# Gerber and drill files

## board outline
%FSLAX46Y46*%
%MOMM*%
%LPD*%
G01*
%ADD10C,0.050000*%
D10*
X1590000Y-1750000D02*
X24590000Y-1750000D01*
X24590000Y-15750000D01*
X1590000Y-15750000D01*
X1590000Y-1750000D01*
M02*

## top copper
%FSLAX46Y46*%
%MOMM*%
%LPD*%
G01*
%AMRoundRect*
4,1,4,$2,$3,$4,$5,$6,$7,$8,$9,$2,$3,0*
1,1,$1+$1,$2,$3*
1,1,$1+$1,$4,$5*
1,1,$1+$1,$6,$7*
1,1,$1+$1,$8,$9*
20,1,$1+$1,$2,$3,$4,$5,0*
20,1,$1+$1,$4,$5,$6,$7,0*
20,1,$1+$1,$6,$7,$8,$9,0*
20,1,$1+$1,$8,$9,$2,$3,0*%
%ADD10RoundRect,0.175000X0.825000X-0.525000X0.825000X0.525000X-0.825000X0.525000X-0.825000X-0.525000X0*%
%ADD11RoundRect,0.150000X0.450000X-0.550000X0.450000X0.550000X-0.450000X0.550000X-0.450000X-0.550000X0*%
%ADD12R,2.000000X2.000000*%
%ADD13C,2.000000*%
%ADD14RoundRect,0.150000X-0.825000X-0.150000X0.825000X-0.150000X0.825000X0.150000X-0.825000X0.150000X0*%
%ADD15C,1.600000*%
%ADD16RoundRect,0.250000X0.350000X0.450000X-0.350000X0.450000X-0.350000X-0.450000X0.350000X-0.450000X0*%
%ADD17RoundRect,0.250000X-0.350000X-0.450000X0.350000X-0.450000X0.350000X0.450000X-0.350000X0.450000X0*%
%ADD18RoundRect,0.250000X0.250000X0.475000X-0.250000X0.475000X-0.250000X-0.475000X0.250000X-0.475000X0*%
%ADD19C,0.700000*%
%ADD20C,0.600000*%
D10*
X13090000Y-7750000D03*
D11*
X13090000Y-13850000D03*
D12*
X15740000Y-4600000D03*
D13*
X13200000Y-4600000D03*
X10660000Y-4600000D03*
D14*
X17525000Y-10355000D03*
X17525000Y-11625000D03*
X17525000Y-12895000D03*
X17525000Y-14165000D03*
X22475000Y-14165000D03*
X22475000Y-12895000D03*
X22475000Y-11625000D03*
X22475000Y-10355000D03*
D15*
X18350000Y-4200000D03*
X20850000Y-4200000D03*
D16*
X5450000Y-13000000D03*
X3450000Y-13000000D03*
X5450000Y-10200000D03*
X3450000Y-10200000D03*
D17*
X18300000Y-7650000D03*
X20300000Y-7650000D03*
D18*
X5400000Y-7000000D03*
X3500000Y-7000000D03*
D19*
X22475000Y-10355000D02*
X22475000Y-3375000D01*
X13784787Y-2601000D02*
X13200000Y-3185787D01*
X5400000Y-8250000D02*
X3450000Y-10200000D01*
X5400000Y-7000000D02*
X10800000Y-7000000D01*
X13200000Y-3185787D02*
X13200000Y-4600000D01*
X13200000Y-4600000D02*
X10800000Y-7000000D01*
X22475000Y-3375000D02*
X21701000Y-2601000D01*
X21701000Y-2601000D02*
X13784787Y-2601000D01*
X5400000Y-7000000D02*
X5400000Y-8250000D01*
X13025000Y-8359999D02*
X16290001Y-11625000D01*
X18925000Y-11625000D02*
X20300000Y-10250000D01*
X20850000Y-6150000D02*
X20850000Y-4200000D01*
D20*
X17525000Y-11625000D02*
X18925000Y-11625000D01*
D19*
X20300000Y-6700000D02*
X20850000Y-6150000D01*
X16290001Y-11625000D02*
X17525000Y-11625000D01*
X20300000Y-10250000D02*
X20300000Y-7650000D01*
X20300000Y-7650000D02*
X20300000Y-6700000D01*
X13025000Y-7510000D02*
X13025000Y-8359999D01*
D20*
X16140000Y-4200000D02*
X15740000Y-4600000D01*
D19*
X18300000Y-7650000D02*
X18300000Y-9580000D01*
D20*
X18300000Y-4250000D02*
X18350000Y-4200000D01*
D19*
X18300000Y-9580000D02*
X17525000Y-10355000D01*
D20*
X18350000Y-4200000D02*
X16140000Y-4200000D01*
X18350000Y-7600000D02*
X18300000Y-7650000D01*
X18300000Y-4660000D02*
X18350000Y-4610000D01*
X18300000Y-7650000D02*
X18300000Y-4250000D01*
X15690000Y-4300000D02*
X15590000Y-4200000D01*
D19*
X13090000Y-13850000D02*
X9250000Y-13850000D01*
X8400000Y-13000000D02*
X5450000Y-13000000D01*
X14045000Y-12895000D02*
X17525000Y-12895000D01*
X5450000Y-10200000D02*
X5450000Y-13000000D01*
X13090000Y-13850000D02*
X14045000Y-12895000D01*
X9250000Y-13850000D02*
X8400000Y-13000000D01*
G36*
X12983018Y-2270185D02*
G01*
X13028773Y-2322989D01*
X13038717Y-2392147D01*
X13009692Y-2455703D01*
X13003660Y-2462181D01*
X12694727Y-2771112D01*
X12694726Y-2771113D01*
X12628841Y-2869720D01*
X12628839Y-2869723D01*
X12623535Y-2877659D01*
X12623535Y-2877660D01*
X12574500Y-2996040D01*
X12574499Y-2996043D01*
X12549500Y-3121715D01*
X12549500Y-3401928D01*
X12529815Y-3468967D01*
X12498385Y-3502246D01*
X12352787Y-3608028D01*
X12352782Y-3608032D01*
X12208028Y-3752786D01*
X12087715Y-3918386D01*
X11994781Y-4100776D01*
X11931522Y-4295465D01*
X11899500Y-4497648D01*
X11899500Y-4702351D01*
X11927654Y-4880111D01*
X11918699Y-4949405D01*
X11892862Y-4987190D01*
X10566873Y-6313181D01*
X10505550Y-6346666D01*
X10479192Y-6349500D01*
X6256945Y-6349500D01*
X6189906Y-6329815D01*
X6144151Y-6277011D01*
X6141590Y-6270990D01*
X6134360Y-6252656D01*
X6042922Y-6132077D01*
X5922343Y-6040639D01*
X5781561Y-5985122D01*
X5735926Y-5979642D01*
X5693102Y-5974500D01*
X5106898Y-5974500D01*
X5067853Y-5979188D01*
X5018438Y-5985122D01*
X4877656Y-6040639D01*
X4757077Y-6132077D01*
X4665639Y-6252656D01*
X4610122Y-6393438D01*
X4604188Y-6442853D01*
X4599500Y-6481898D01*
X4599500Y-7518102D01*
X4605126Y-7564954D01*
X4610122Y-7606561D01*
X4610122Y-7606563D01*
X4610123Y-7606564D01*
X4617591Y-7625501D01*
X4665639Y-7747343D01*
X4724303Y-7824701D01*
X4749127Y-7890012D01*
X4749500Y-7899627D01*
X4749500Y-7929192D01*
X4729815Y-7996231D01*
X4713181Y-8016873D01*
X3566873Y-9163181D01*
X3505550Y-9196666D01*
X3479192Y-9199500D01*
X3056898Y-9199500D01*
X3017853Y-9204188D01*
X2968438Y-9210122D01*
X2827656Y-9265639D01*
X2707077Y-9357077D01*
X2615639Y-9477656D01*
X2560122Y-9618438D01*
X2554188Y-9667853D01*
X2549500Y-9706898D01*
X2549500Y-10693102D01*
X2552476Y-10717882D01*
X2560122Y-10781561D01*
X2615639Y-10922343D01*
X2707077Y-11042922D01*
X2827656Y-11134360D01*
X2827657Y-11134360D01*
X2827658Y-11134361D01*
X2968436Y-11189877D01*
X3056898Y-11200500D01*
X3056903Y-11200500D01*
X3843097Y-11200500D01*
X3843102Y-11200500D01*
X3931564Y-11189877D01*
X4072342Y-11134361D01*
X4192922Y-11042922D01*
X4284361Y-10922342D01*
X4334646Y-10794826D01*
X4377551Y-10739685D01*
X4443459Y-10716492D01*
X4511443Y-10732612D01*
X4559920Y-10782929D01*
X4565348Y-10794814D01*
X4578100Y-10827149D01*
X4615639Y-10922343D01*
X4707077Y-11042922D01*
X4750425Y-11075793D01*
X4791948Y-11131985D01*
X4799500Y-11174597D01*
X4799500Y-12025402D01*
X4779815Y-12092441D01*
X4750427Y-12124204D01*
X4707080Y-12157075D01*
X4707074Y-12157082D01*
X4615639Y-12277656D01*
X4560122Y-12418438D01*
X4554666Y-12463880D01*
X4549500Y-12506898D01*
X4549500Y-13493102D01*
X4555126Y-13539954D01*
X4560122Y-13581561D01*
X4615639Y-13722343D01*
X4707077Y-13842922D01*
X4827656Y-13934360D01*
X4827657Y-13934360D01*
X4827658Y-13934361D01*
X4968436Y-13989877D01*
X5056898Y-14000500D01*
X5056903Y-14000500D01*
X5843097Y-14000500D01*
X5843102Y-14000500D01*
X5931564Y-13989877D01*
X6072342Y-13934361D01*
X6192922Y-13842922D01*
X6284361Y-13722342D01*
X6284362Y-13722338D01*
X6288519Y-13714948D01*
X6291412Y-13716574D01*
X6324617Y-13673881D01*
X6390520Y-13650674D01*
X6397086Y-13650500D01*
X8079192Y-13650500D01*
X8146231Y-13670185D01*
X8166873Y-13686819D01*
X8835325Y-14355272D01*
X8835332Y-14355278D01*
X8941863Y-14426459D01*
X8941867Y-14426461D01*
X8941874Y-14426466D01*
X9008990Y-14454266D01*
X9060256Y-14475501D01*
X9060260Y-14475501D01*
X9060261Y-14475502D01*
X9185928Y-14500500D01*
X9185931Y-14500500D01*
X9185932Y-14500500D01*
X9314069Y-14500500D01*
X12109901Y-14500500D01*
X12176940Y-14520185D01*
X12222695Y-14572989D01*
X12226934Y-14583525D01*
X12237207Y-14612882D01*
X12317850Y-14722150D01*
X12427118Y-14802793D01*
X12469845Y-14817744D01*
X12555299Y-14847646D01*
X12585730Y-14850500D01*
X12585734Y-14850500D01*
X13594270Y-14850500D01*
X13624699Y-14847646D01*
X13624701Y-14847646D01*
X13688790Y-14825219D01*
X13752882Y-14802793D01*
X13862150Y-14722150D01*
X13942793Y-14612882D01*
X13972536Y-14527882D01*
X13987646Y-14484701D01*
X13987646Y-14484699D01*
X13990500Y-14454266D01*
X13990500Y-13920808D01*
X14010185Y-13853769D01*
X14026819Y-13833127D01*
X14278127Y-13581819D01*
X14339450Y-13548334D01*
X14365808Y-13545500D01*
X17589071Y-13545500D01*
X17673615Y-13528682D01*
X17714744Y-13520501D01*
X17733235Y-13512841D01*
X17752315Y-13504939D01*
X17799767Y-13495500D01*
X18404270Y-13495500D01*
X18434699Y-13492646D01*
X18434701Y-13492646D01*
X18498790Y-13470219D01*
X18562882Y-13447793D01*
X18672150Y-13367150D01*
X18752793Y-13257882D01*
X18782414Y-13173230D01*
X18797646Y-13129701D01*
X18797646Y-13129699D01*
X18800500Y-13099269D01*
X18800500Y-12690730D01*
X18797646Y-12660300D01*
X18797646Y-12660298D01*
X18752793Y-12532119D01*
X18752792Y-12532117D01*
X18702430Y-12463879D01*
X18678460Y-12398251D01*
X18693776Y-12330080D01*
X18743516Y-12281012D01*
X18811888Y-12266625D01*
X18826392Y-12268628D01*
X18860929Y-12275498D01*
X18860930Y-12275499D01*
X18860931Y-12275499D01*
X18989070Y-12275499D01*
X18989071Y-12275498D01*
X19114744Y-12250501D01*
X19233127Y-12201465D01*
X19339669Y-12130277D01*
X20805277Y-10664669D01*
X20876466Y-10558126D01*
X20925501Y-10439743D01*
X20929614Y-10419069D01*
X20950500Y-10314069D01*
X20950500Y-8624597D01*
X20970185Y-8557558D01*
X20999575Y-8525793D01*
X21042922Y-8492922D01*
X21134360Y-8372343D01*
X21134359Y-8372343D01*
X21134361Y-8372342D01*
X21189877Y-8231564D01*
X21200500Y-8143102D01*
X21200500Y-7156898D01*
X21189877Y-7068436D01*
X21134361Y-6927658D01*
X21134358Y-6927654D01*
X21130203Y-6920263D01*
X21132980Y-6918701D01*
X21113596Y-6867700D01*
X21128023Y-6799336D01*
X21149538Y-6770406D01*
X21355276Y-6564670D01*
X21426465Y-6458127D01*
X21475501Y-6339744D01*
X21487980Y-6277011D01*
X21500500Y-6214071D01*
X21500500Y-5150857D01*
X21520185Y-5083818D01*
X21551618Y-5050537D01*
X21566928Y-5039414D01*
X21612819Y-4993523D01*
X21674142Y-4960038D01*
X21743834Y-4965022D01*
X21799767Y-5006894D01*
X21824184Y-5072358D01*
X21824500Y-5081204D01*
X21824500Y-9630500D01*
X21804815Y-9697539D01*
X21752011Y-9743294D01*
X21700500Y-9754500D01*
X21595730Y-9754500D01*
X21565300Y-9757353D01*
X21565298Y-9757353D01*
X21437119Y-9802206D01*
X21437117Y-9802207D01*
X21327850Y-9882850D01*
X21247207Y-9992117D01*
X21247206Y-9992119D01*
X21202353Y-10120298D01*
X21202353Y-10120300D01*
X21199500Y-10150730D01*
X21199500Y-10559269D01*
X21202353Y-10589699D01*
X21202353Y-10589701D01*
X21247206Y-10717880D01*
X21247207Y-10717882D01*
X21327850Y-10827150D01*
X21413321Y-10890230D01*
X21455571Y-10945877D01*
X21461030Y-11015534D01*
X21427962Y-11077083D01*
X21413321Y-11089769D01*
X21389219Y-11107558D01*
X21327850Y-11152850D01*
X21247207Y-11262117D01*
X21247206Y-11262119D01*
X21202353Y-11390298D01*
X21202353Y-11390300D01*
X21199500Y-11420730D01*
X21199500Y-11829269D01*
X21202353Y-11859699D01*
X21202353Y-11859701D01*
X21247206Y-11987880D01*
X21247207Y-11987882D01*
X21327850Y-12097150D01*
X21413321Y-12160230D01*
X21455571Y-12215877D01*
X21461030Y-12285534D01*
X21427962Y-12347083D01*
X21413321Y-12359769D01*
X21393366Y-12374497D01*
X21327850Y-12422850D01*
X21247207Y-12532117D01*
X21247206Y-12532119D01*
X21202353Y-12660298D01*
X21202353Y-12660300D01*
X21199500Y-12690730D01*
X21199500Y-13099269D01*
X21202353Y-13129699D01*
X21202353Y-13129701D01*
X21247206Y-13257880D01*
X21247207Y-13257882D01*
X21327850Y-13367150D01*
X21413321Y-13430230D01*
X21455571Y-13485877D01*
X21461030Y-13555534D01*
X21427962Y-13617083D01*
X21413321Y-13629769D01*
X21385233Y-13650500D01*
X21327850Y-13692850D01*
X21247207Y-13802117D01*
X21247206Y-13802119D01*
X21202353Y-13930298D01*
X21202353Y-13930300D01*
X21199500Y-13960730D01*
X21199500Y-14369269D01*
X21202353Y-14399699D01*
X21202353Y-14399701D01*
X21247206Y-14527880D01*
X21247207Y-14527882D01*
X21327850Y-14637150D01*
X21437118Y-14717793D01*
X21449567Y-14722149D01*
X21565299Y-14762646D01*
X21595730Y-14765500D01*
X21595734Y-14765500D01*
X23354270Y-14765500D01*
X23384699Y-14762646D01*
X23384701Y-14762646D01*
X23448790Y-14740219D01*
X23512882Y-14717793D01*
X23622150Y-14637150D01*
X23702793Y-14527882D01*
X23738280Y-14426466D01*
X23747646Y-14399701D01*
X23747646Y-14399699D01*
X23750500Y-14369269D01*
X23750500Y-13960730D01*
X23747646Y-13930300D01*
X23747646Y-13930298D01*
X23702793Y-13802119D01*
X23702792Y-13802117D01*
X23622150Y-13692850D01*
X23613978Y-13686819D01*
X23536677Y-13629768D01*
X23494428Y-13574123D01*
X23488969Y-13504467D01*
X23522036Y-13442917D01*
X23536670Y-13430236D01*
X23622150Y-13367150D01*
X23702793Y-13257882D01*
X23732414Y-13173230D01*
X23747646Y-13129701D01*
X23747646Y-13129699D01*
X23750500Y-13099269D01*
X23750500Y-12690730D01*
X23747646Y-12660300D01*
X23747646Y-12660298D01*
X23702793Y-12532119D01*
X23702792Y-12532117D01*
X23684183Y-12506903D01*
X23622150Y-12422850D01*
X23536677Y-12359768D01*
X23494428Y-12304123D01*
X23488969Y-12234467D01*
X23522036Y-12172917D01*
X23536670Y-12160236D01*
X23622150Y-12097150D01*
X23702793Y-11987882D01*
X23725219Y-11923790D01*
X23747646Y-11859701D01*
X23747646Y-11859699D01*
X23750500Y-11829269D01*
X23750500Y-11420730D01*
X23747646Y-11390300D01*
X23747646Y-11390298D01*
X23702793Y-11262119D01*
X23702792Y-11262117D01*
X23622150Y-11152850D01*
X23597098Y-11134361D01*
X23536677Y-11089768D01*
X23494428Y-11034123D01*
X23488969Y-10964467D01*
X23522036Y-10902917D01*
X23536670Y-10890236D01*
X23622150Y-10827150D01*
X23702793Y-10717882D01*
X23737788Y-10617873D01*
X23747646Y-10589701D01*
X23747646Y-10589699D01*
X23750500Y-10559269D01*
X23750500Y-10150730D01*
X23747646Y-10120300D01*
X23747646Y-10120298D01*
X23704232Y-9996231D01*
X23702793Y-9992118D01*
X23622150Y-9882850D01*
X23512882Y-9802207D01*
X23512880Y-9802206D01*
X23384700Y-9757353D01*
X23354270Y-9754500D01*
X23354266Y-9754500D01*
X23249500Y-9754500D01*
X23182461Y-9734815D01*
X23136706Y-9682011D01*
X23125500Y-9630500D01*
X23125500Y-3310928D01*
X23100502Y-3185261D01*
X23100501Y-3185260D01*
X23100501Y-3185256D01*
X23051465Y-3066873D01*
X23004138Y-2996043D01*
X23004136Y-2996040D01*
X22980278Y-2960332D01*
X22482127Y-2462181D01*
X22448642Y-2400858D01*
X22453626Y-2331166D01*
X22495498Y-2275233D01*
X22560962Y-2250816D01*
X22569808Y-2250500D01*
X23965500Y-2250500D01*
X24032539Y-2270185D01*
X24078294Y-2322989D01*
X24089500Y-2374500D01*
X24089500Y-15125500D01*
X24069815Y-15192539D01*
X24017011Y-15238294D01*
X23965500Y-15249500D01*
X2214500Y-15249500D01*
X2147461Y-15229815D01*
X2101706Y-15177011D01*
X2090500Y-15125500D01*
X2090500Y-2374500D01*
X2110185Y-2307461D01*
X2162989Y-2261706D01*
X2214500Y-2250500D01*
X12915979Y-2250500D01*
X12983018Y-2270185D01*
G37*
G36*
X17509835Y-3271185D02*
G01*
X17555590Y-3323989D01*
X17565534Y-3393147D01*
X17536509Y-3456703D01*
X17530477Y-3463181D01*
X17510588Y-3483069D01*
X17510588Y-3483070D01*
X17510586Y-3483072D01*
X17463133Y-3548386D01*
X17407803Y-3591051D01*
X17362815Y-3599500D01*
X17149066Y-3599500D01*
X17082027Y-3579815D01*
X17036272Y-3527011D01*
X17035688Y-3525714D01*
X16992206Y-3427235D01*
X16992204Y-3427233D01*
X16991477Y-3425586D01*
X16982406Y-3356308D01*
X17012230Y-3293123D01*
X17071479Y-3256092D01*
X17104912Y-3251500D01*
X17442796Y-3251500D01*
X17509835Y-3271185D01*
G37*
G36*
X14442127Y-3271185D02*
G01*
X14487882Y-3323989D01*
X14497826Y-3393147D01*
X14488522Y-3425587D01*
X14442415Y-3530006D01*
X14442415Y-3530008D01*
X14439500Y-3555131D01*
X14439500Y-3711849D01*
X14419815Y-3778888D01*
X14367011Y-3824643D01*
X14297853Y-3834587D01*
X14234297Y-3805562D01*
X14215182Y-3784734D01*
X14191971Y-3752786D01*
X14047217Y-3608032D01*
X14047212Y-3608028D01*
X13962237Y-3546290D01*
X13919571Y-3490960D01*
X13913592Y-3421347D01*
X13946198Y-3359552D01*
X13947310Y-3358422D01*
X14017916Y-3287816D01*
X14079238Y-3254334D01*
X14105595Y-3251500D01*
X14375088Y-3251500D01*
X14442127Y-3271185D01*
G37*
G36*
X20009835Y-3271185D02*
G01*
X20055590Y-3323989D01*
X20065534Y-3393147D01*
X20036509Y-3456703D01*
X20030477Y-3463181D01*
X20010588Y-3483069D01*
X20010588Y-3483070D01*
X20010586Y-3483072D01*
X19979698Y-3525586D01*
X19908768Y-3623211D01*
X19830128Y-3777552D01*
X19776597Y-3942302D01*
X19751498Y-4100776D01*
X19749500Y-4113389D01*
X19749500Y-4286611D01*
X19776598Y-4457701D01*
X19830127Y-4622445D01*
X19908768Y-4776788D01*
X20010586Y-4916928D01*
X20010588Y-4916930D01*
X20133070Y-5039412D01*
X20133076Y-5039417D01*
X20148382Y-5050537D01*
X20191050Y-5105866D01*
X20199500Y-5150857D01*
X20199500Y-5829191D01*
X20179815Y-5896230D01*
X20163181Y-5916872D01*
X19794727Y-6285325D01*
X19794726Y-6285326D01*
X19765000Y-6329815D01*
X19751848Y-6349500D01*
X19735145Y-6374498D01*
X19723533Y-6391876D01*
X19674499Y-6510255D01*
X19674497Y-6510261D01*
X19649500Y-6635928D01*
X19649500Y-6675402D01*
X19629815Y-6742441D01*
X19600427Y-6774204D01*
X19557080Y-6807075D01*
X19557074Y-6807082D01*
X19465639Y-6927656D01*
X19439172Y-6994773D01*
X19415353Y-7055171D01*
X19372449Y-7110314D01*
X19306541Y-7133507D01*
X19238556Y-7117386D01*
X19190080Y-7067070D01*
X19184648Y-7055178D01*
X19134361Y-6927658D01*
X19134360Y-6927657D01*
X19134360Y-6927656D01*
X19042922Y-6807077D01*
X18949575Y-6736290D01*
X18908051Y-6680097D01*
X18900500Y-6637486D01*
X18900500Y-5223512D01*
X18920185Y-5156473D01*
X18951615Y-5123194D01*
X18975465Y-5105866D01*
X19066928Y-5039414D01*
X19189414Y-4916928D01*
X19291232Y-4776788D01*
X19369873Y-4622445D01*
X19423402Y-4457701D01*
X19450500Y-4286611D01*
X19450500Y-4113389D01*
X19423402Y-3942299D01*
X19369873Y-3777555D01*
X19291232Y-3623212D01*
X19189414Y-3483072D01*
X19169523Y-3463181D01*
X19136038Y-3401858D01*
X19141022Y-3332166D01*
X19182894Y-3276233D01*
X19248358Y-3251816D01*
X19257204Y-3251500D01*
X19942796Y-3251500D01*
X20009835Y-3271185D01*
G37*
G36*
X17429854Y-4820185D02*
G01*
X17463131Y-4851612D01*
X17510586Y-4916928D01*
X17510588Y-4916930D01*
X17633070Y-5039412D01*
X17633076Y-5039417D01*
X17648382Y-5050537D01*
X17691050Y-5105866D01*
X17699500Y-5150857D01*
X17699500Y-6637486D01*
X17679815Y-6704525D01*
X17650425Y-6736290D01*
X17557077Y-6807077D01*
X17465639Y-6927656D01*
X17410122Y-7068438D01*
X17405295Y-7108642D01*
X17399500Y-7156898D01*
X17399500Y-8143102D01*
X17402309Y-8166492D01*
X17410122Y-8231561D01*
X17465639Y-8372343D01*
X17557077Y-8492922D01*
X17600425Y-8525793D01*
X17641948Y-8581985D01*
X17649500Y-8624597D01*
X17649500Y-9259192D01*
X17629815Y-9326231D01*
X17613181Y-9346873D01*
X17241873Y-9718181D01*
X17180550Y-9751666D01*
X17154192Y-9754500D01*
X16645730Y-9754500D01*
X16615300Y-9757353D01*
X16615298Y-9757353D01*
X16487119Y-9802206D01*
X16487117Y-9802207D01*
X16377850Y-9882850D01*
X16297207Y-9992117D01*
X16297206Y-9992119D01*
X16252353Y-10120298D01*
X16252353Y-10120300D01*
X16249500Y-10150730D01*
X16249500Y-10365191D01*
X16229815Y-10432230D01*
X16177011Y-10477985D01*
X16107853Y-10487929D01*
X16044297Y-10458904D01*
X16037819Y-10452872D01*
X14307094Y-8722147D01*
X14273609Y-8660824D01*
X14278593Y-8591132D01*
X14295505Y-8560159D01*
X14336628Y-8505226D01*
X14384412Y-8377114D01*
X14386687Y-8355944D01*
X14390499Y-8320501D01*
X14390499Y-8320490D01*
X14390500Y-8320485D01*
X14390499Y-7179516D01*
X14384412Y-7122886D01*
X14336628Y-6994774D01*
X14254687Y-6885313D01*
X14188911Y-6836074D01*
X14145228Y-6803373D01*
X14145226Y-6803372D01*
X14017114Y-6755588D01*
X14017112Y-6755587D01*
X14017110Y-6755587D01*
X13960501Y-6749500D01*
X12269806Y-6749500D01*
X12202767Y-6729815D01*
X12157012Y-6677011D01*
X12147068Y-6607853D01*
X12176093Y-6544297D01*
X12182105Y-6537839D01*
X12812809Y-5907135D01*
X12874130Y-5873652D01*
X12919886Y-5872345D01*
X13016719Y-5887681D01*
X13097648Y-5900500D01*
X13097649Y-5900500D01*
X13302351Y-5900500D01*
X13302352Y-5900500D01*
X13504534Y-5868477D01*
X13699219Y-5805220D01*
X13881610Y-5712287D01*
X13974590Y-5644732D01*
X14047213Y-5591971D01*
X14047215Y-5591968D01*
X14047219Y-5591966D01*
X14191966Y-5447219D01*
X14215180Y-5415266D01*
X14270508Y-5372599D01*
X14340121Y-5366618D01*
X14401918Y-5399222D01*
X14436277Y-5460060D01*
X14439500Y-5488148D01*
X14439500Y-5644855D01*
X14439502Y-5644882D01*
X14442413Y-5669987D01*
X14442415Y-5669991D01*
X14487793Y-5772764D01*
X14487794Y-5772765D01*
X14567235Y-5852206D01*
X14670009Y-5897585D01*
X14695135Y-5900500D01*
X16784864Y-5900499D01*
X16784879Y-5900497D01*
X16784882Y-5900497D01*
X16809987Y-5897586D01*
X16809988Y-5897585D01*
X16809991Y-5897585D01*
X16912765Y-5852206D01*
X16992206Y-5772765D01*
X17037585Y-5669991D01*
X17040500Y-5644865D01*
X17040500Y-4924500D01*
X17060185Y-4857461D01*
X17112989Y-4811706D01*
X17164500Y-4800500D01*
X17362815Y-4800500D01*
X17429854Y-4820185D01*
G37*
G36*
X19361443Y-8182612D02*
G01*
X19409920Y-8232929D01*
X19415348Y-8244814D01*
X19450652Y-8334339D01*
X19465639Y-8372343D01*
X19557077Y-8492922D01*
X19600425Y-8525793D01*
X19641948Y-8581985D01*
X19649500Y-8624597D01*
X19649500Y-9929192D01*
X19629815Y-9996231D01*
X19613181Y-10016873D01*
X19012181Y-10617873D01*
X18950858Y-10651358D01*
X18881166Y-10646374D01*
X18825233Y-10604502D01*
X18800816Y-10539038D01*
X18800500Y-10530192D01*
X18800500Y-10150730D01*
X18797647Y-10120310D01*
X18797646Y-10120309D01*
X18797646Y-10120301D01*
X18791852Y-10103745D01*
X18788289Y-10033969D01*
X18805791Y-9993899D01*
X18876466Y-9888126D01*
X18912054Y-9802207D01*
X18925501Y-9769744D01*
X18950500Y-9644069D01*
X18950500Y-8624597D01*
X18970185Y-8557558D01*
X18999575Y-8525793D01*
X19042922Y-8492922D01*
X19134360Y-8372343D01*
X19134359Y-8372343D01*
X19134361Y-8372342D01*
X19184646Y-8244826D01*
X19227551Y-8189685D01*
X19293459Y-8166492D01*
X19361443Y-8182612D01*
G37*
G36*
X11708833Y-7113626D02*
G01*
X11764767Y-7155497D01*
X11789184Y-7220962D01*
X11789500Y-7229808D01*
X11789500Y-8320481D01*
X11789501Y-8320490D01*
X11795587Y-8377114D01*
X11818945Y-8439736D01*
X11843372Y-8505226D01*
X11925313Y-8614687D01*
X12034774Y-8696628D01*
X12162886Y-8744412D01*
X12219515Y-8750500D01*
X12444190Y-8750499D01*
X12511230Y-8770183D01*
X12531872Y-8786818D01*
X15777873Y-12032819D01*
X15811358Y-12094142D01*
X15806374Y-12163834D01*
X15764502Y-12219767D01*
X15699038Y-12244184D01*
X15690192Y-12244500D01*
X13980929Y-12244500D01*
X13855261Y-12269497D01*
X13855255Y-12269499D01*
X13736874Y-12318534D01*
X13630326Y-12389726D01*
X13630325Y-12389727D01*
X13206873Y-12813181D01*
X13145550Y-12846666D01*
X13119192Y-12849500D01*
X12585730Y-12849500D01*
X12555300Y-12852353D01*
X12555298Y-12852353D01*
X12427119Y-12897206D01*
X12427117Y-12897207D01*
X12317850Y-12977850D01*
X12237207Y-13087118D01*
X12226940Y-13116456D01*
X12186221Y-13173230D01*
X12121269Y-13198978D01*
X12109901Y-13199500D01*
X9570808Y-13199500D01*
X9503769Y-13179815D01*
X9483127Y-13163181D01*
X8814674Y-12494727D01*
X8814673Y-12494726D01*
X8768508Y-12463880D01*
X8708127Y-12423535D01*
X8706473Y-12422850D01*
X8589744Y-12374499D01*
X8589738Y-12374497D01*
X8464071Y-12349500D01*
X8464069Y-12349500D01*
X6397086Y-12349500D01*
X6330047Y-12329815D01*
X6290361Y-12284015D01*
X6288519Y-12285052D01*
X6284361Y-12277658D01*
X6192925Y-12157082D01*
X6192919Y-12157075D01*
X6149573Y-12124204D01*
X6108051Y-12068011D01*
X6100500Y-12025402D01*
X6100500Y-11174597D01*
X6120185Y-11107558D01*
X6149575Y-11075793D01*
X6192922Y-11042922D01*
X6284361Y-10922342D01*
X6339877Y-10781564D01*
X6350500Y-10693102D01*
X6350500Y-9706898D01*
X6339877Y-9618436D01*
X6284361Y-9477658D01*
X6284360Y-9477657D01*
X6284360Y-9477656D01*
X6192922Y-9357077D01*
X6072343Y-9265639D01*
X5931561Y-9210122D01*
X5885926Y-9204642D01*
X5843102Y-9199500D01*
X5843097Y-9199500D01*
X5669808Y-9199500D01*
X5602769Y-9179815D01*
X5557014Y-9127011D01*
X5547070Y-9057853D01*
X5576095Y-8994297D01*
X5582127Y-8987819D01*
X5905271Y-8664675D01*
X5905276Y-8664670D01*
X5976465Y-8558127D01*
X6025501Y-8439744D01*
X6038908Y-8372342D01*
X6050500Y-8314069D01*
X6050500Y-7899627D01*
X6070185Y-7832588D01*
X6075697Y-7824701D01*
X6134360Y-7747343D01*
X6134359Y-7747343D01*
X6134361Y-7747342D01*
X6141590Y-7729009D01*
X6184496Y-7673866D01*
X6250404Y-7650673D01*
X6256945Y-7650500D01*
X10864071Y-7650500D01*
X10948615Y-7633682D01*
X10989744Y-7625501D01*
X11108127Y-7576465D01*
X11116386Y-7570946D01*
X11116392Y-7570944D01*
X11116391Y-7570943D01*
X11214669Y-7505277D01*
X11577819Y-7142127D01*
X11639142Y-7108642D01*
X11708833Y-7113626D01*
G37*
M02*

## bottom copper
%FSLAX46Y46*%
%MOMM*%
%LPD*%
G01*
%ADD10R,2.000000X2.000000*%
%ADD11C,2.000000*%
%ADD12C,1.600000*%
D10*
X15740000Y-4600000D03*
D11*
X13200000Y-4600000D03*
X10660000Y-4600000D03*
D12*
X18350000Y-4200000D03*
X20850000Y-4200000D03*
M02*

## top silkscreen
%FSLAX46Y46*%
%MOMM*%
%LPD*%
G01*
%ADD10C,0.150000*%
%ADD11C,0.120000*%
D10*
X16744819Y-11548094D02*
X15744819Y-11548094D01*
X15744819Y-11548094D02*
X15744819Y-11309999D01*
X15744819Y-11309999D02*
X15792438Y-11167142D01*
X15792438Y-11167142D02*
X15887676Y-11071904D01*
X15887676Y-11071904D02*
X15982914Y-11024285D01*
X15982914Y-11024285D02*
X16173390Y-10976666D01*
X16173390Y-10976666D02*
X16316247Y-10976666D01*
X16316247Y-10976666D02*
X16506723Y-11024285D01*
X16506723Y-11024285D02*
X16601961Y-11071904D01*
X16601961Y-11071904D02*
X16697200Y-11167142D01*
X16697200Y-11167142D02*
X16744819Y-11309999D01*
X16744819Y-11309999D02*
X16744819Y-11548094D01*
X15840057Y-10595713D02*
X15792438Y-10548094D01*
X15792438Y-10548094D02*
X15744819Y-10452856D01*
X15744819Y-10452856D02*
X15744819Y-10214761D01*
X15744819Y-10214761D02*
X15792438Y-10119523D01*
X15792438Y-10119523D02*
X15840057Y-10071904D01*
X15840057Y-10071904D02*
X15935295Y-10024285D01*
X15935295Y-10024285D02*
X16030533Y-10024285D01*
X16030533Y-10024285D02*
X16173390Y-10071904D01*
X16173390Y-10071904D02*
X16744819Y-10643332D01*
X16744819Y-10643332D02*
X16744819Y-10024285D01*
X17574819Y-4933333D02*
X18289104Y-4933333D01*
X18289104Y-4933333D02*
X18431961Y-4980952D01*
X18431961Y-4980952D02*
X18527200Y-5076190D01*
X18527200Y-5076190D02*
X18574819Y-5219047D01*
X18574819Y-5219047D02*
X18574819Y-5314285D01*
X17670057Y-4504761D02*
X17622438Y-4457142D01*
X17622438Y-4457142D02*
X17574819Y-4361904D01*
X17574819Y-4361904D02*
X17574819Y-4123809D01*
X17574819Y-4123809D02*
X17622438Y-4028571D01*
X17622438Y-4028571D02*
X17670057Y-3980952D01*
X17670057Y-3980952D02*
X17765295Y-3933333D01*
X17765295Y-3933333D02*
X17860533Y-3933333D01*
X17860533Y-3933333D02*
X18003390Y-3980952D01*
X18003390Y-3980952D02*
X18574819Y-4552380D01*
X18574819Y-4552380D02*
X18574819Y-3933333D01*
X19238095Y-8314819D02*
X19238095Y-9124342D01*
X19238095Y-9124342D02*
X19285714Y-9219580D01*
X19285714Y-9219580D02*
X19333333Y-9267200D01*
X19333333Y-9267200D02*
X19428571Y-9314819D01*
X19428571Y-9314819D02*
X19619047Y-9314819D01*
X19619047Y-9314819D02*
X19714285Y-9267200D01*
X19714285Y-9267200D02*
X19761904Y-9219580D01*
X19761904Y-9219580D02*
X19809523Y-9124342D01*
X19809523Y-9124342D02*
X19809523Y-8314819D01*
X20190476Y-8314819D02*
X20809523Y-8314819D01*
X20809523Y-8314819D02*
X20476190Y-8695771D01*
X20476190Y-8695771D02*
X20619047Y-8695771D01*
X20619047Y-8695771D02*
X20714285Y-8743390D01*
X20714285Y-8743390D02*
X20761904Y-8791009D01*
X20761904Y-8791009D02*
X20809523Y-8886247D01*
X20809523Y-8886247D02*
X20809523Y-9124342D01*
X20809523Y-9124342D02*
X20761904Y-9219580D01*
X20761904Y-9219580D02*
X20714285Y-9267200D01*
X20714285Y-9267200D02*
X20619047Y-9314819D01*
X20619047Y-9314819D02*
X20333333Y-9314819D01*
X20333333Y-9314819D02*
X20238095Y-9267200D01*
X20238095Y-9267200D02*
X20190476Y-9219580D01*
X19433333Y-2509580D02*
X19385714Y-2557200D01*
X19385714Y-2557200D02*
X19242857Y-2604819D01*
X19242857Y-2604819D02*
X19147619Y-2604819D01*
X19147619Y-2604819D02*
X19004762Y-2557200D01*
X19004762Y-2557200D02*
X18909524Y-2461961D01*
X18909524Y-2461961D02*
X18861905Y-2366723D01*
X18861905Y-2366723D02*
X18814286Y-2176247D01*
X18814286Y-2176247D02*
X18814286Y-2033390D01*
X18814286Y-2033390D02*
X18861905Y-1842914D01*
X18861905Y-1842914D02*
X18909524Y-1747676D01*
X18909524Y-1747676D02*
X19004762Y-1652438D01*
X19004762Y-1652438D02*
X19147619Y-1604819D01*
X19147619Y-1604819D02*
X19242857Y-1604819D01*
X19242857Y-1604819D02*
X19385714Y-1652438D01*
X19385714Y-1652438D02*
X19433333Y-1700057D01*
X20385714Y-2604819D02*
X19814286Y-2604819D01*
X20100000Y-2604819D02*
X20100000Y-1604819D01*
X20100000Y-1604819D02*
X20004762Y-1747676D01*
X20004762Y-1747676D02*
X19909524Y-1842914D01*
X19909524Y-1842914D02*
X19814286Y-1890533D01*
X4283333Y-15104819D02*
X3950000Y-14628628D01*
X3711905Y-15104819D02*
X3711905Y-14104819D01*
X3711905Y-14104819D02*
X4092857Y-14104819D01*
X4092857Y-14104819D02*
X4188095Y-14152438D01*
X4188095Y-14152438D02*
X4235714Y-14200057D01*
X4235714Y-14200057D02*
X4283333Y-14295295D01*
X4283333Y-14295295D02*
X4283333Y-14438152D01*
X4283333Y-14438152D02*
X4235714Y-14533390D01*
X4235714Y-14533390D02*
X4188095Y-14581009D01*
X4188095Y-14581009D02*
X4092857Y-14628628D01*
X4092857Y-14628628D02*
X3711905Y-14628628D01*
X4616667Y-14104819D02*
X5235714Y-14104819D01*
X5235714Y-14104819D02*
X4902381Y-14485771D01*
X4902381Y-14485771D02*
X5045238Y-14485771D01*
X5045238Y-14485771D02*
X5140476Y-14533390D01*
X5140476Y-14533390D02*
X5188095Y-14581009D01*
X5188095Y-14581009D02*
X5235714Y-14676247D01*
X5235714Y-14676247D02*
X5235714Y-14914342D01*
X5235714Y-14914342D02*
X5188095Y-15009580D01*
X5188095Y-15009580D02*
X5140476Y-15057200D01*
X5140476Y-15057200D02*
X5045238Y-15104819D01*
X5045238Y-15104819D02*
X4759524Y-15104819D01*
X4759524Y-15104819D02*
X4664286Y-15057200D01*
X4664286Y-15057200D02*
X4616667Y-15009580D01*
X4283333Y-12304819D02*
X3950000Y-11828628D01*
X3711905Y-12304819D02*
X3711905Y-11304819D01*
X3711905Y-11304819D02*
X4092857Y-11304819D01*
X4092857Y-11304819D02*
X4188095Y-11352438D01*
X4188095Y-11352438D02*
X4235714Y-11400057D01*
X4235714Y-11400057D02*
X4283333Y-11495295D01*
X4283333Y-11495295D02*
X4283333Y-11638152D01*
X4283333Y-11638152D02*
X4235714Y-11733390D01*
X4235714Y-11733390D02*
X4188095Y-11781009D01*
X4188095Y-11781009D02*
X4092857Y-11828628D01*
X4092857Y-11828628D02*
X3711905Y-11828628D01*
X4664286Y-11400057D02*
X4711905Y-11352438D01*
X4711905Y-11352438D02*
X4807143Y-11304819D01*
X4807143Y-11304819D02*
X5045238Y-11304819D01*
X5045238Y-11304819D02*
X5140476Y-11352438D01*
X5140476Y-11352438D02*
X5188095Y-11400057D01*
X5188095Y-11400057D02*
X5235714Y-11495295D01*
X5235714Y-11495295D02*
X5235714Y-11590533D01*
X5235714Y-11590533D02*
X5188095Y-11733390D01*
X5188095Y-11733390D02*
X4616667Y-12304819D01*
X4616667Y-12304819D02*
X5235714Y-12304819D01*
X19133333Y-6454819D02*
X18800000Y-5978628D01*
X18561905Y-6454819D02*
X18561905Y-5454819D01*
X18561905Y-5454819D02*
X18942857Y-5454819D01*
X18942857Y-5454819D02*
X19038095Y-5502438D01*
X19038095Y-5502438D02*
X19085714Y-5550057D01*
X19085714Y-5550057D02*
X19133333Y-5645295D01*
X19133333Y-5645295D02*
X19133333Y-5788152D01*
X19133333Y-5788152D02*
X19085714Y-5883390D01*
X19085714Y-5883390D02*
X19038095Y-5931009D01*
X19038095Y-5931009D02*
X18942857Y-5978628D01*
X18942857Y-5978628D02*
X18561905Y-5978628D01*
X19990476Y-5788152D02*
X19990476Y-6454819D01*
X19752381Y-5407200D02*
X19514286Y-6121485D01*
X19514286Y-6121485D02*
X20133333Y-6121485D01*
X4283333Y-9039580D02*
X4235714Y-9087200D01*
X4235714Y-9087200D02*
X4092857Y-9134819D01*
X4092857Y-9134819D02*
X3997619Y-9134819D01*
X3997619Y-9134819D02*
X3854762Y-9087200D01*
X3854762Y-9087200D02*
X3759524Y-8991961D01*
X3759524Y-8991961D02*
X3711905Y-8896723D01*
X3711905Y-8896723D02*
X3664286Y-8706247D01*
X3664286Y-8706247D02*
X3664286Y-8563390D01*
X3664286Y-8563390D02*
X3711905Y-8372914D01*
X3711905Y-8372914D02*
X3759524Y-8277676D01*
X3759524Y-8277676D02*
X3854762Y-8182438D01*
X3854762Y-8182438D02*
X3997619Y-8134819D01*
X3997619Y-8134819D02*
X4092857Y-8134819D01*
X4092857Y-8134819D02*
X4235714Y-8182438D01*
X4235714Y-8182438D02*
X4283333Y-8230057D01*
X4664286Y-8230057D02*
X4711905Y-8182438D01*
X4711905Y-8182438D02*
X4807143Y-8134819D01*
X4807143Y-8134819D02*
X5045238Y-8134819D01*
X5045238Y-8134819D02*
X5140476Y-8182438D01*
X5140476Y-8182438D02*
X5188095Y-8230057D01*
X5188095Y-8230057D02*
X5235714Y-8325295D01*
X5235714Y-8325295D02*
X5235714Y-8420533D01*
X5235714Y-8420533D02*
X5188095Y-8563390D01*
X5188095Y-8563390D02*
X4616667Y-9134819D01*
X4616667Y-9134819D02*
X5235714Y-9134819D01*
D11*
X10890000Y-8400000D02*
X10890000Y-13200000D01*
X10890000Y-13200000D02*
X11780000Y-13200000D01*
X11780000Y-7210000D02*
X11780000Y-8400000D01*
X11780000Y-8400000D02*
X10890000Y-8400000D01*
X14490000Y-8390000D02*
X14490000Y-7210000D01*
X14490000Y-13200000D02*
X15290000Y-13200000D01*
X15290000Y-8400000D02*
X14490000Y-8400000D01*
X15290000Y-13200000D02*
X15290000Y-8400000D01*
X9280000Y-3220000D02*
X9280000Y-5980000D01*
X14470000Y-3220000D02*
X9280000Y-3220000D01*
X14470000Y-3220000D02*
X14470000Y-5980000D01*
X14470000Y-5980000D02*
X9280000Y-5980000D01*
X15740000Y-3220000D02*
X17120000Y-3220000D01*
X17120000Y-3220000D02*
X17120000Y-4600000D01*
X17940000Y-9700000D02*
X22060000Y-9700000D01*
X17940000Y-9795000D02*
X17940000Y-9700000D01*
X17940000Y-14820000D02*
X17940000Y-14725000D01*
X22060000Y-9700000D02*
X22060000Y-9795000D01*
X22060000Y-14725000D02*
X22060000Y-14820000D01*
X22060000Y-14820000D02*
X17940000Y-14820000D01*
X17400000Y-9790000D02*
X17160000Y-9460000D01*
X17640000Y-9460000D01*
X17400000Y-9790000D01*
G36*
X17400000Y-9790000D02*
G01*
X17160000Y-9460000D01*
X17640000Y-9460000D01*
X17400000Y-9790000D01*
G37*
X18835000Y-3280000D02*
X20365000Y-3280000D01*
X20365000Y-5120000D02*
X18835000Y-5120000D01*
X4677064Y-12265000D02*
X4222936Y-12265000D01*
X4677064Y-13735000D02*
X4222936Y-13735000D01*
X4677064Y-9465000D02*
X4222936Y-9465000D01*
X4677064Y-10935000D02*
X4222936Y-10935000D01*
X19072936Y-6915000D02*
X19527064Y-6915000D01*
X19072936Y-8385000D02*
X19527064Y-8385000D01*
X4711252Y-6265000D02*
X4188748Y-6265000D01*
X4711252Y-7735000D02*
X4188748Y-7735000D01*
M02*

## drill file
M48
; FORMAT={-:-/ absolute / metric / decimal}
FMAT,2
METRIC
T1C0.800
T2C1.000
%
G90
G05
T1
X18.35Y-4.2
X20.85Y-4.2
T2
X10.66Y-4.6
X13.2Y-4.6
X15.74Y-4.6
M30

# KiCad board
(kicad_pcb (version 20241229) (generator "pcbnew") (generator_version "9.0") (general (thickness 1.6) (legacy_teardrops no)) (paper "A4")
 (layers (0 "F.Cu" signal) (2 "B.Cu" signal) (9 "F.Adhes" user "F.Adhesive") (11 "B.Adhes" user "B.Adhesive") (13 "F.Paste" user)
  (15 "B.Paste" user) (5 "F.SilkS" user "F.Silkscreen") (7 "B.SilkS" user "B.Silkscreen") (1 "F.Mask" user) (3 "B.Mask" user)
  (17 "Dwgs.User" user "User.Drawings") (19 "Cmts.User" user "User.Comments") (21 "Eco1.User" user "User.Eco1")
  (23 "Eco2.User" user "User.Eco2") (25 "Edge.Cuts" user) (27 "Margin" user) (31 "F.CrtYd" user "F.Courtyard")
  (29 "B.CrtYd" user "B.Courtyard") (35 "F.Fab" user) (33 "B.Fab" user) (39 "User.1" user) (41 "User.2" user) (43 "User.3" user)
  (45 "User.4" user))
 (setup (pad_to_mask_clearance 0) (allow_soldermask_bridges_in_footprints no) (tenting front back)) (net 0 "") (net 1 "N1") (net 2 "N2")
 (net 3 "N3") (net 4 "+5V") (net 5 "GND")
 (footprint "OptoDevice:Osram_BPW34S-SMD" (layer "F.Cu") (at 13.09 10.8 -90)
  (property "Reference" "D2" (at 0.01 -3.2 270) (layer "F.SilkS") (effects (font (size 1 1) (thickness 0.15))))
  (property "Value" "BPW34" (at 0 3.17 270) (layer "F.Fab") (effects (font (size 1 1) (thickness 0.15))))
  (fp_line (start -2.4 2.2) (end 2.4 2.2) (stroke (width 0.12) (type solid)) (layer "F.SilkS"))
  (fp_line (start 2.4 2.2) (end 2.4 1.31) (stroke (width 0.12) (type solid)) (layer "F.SilkS"))
  (fp_line (start -3.59 1.31) (end -2.4 1.31) (stroke (width 0.12) (type solid)) (layer "F.SilkS"))
  (fp_line (start -2.4 1.31) (end -2.4 2.2) (stroke (width 0.12) (type solid)) (layer "F.SilkS"))
  (fp_line (start -2.41 -1.4) (end -3.59 -1.4) (stroke (width 0.12) (type solid)) (layer "F.SilkS"))
  (fp_line (start 2.4 -1.4) (end 2.4 -2.2) (stroke (width 0.12) (type solid)) (layer "F.SilkS"))
  (fp_line (start -2.4 -2.2) (end -2.4 -1.4) (stroke (width 0.12) (type solid)) (layer "F.SilkS"))
  (fp_line (start 2.4 -2.2) (end -2.4 -2.2) (stroke (width 0.12) (type solid)) (layer "F.SilkS"))
  (pad "" smd roundrect (at -3.05 0 90) (size 1.3 1.9) (layers "F.Paste") (roundrect_rratio 0.125))
  (pad "" smd roundrect (at -3.05 0 90) (size 1.5 2.1) (layers "F.Mask") (roundrect_rratio 0.125))
  (pad "" smd roundrect (at 3.05 0 90) (size 1.3 1.1) (layers "F.Paste") (roundrect_rratio 0.125))
  (pad "" smd roundrect (at 3.05 0 90) (size 1.5 1.3) (layers "F.Mask") (roundrect_rratio 0.125))
  (pad "1" smd roundrect (at -3.05 0 90) (size 1.4 2) (layers "F.Cu" "F.Mask") (roundrect_rratio 0.125) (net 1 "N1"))
  (pad "2" smd roundrect (at 3.05 0 90) (size 1.4 1.2) (layers "F.Cu" "F.Mask") (roundrect_rratio 0.125) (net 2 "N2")))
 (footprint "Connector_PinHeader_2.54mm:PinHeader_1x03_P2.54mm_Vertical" (layer "F.Cu") (at 15.74 4.6 -90)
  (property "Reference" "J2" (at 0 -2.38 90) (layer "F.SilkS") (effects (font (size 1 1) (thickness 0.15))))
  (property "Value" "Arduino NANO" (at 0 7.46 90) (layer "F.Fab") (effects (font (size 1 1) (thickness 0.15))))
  (fp_line (start -1.38 6.46) (end 1.38 6.46) (stroke (width 0.12) (type solid)) (layer "F.SilkS"))
  (fp_line (start -1.38 1.27) (end -1.38 6.46) (stroke (width 0.12) (type solid)) (layer "F.SilkS"))
  (fp_line (start -1.38 1.27) (end 1.38 1.27) (stroke (width 0.12) (type solid)) (layer "F.SilkS"))
  (fp_line (start 1.38 1.27) (end 1.38 6.46) (stroke (width 0.12) (type solid)) (layer "F.SilkS"))
  (fp_line (start -1.38 0) (end -1.38 -1.38) (stroke (width 0.12) (type solid)) (layer "F.SilkS"))
  (fp_line (start -1.38 -1.38) (end 0 -1.38) (stroke (width 0.12) (type solid)) (layer "F.SilkS"))
  (pad "1" thru_hole rect (at 0 0 270) (size 2 2) (drill 1) (layers "*.Cu" "*.Mask") (remove_unused_layers no) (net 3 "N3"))
  (pad "2" thru_hole circle (at 0 2.54 270) (size 2 2) (drill 1) (layers "*.Cu" "*.Mask") (remove_unused_layers no) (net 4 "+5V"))
  (pad "3" thru_hole circle (at 0 5.08 270) (size 2 2) (drill 1) (layers "*.Cu" "*.Mask") (remove_unused_layers no) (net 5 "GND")))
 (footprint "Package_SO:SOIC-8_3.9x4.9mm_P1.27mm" (layer "F.Cu") (at 20 12.26)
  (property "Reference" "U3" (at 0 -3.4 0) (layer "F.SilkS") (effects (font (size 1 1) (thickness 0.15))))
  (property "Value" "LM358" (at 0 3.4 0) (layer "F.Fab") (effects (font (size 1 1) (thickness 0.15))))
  (fp_line (start -2.06 -2.56) (end 2.06 -2.56) (stroke (width 0.12) (type solid)) (layer "F.SilkS"))
  (fp_line (start -2.06 -2.465) (end -2.06 -2.56) (stroke (width 0.12) (type solid)) (layer "F.SilkS"))
  (fp_line (start -2.06 2.56) (end -2.06 2.465) (stroke (width 0.12) (type solid)) (layer "F.SilkS"))
  (fp_line (start 2.06 -2.56) (end 2.06 -2.465) (stroke (width 0.12) (type solid)) (layer "F.SilkS"))
  (fp_line (start 2.06 2.465) (end 2.06 2.56) (stroke (width 0.12) (type solid)) (layer "F.SilkS"))
  (fp_line (start 2.06 2.56) (end -2.06 2.56) (stroke (width 0.12) (type solid)) (layer "F.SilkS"))
  (fp_poly (pts (xy -2.6 -2.47) (xy -2.84 -2.8) (xy -2.36 -2.8)) (stroke (width 0.12) (type solid)) (fill yes) (layer "F.SilkS"))
  (pad "1" smd roundrect (at -2.475 -1.905) (size 1.95 0.6) (layers "F.Cu" "F.Mask" "F.Paste") (roundrect_rratio 0.25) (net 3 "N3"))
  (pad "2" smd roundrect (at -2.475 -0.635) (size 1.95 0.6) (layers "F.Cu" "F.Mask" "F.Paste") (roundrect_rratio 0.25) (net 1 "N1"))
  (pad "3" smd roundrect (at -2.475 0.635) (size 1.95 0.6) (layers "F.Cu" "F.Mask" "F.Paste") (roundrect_rratio 0.25) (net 2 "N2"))
  (pad "4" smd roundrect (at -2.475 1.905) (size 1.95 0.6) (layers "F.Cu" "F.Mask" "F.Paste") (roundrect_rratio 0.25) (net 5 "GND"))
  (pad "5" smd roundrect (at 2.475 1.905) (size 1.95 0.6) (layers "F.Cu" "F.Mask" "F.Paste") (roundrect_rratio 0.25))
  (pad "6" smd roundrect (at 2.475 0.635) (size 1.95 0.6) (layers "F.Cu" "F.Mask" "F.Paste") (roundrect_rratio 0.25))
  (pad "7" smd roundrect (at 2.475 -0.635) (size 1.95 0.6) (layers "F.Cu" "F.Mask" "F.Paste") (roundrect_rratio 0.25))
  (pad "8" smd roundrect (at 2.475 -1.905) (size 1.95 0.6) (layers "F.Cu" "F.Mask" "F.Paste") (roundrect_rratio 0.25) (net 4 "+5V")))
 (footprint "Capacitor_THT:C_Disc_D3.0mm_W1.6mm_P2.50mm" (layer "F.Cu") (at 18.35 4.2)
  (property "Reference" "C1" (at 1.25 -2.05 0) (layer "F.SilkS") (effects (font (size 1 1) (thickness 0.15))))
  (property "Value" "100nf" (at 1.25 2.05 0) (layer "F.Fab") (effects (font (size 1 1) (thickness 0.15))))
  (fp_line (start 0.485 -0.92) (end 2.015 -0.92) (stroke (width 0.12) (type solid)) (layer "F.SilkS"))
  (fp_line (start 2.015 0.92) (end 0.485 0.92) (stroke (width 0.12) (type solid)) (layer "F.SilkS"))
  (pad "1" thru_hole circle (at 0 0) (size 1.6 1.6) (drill 0.8) (layers "*.Cu" "*.Mask") (remove_unused_layers no) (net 3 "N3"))
  (pad "2" thru_hole circle (at 2.5 0) (size 1.6 1.6) (drill 0.8) (layers "*.Cu" "*.Mask") (remove_unused_layers no) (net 1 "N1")))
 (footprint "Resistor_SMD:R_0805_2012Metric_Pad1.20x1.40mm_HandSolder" (layer "F.Cu") (at 4.45 13 180)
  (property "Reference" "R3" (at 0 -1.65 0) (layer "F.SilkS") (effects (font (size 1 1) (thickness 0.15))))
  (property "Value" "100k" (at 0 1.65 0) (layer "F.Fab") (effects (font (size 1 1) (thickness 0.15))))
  (fp_line (start -0.227064 0.735) (end 0.227064 0.735) (stroke (width 0.12) (type solid)) (layer "F.SilkS"))
  (fp_line (start -0.227064 -0.735) (end 0.227064 -0.735) (stroke (width 0.12) (type solid)) (layer "F.SilkS"))
  (pad "1" smd roundrect (at -1 0 180) (size 1.2 1.4) (layers "F.Cu" "F.Mask" "F.Paste") (roundrect_rratio 0.208333) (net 2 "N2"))
  (pad "2" smd roundrect (at 1 0 180) (size 1.2 1.4) (layers "F.Cu" "F.Mask" "F.Paste") (roundrect_rratio 0.208333) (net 5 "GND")))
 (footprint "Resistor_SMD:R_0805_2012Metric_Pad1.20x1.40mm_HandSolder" (layer "F.Cu") (at 4.45 10.2 180)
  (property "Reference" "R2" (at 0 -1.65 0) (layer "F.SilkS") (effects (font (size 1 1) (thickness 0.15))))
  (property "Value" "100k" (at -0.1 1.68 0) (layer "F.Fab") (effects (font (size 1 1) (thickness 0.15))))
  (fp_line (start -0.227064 0.735) (end 0.227064 0.735) (stroke (width 0.12) (type solid)) (layer "F.SilkS"))
  (fp_line (start -0.227064 -0.735) (end 0.227064 -0.735) (stroke (width 0.12) (type solid)) (layer "F.SilkS"))
  (pad "1" smd roundrect (at -1 0 180) (size 1.2 1.4) (layers "F.Cu" "F.Mask" "F.Paste") (roundrect_rratio 0.208333) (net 2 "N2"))
  (pad "2" smd roundrect (at 1 0 180) (size 1.2 1.4) (layers "F.Cu" "F.Mask" "F.Paste") (roundrect_rratio 0.208333) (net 4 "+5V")))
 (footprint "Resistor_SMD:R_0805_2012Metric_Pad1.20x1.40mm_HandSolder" (layer "F.Cu") (at 19.3 7.65)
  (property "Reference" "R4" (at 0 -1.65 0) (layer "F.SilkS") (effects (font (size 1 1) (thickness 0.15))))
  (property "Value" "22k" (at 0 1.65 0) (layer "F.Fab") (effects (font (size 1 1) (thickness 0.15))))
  (fp_line (start -0.227064 -0.735) (end 0.227064 -0.735) (stroke (width 0.12) (type solid)) (layer "F.SilkS"))
  (fp_line (start -0.227064 0.735) (end 0.227064 0.735) (stroke (width 0.12) (type solid)) (layer "F.SilkS"))
  (pad "1" smd roundrect (at -1 0) (size 1.2 1.4) (layers "F.Cu" "F.Mask" "F.Paste") (roundrect_rratio 0.208333) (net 3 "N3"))
  (pad "2" smd roundrect (at 1 0) (size 1.2 1.4) (layers "F.Cu" "F.Mask" "F.Paste") (roundrect_rratio 0.208333) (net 1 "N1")))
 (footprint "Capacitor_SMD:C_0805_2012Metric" (layer "F.Cu") (at 4.45 7 180)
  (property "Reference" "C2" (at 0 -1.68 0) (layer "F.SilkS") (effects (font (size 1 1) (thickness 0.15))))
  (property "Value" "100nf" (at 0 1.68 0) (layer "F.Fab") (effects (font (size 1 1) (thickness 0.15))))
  (fp_line (start -0.261252 0.735) (end 0.261252 0.735) (stroke (width 0.12) (type solid)) (layer "F.SilkS"))
  (fp_line (start -0.261252 -0.735) (end 0.261252 -0.735) (stroke (width 0.12) (type solid)) (layer "F.SilkS"))
  (pad "1" smd roundrect (at -0.95 0 180) (size 1 1.45) (layers "F.Cu" "F.Mask" "F.Paste") (roundrect_rratio 0.25) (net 4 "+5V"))
  (pad "2" smd roundrect (at 0.95 0 180) (size 1 1.45) (layers "F.Cu" "F.Mask" "F.Paste") (roundrect_rratio 0.25) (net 5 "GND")))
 (gr_rect (start 1.59 1.75) (end 24.59 15.75) (stroke (width 0.05) (type default)) (fill no) (layer "Edge.Cuts"))
 (segment (start 22.475 10.355) (end 22.475 3.375) (width 0.7) (layer "F.Cu") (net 4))
 (segment (start 13.784787 2.601) (end 13.2 3.185787) (width 0.7) (layer "F.Cu") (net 4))
 (segment (start 5.4 8.25) (end 3.45 10.2) (width 0.7) (layer "F.Cu") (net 4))
 (segment (start 5.4 7) (end 10.8 7) (width 0.7) (layer "F.Cu") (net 4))
 (segment (start 13.2 3.185787) (end 13.2 4.6) (width 0.7) (layer "F.Cu") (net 4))
 (segment (start 13.2 4.6) (end 10.8 7) (width 0.7) (layer "F.Cu") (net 4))
 (segment (start 22.475 3.375) (end 21.701 2.601) (width 0.7) (layer "F.Cu") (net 4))
 (segment (start 21.701 2.601) (end 13.784787 2.601) (width 0.7) (layer "F.Cu") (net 4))
 (segment (start 5.4 7) (end 5.4 8.25) (width 0.7) (layer "F.Cu") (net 4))
 (segment (start 13.025 8.359999) (end 16.290001 11.625) (width 0.7) (layer "F.Cu") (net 1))
 (segment (start 18.925 11.625) (end 20.3 10.25) (width 0.7) (layer "F.Cu") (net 1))
 (segment (start 20.85 6.15) (end 20.85 4.2) (width 0.7) (layer "F.Cu") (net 1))
 (segment (start 17.525 11.625) (end 18.925 11.625) (width 0.6) (layer "F.Cu") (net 1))
 (segment (start 20.3 6.7) (end 20.85 6.15) (width 0.7) (layer "F.Cu") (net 1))
 (segment (start 16.290001 11.625) (end 17.525 11.625) (width 0.7) (layer "F.Cu") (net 1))
 (segment (start 20.3 10.25) (end 20.3 7.65) (width 0.7) (layer "F.Cu") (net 1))
 (segment (start 20.3 7.65) (end 20.3 6.7) (width 0.7) (layer "F.Cu") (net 1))
 (segment (start 13.025 7.51) (end 13.025 8.359999) (width 0.7) (layer "F.Cu") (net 1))
 (segment (start 16.14 4.2) (end 15.74 4.6) (width 0.6) (layer "F.Cu") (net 3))
 (segment (start 18.3 7.65) (end 18.3 9.58) (width 0.7) (layer "F.Cu") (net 3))
 (segment (start 18.3 4.25) (end 18.35 4.2) (width 0.6) (layer "F.Cu") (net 3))
 (segment (start 18.3 9.58) (end 17.525 10.355) (width 0.7) (layer "F.Cu") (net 3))
 (segment (start 18.35 4.2) (end 16.14 4.2) (width 0.6) (layer "F.Cu") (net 3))
 (segment (start 18.35 7.6) (end 18.3 7.65) (width 0.6) (layer "F.Cu") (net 3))
 (segment (start 18.3 4.66) (end 18.35 4.61) (width 0.6) (layer "F.Cu") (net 3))
 (segment (start 18.3 7.65) (end 18.3 4.25) (width 0.6) (layer "F.Cu") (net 3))
 (segment (start 15.69 4.3) (end 15.59 4.2) (width 0.6) (layer "F.Cu") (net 3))
 (segment (start 13.09 13.85) (end 9.25 13.85) (width 0.7) (layer "F.Cu") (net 2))
 (segment (start 8.4 13) (end 5.45 13) (width 0.7) (layer "F.Cu") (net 2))
 (segment (start 14.045 12.895) (end 17.525 12.895) (width 0.7) (layer "F.Cu") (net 2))
 (segment (start 5.45 10.2) (end 5.45 13) (width 0.7) (layer "F.Cu") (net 2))
 (segment (start 13.09 13.85) (end 14.045 12.895) (width 0.7) (layer "F.Cu") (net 2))
 (segment (start 9.25 13.85) (end 8.4 13) (width 0.7) (layer "F.Cu") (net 2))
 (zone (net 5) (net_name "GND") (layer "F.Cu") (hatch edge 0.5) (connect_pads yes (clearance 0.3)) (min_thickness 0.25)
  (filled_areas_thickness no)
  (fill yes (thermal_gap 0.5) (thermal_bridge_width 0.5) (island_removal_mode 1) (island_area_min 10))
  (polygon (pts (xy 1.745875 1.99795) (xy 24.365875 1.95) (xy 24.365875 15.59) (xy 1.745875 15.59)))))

